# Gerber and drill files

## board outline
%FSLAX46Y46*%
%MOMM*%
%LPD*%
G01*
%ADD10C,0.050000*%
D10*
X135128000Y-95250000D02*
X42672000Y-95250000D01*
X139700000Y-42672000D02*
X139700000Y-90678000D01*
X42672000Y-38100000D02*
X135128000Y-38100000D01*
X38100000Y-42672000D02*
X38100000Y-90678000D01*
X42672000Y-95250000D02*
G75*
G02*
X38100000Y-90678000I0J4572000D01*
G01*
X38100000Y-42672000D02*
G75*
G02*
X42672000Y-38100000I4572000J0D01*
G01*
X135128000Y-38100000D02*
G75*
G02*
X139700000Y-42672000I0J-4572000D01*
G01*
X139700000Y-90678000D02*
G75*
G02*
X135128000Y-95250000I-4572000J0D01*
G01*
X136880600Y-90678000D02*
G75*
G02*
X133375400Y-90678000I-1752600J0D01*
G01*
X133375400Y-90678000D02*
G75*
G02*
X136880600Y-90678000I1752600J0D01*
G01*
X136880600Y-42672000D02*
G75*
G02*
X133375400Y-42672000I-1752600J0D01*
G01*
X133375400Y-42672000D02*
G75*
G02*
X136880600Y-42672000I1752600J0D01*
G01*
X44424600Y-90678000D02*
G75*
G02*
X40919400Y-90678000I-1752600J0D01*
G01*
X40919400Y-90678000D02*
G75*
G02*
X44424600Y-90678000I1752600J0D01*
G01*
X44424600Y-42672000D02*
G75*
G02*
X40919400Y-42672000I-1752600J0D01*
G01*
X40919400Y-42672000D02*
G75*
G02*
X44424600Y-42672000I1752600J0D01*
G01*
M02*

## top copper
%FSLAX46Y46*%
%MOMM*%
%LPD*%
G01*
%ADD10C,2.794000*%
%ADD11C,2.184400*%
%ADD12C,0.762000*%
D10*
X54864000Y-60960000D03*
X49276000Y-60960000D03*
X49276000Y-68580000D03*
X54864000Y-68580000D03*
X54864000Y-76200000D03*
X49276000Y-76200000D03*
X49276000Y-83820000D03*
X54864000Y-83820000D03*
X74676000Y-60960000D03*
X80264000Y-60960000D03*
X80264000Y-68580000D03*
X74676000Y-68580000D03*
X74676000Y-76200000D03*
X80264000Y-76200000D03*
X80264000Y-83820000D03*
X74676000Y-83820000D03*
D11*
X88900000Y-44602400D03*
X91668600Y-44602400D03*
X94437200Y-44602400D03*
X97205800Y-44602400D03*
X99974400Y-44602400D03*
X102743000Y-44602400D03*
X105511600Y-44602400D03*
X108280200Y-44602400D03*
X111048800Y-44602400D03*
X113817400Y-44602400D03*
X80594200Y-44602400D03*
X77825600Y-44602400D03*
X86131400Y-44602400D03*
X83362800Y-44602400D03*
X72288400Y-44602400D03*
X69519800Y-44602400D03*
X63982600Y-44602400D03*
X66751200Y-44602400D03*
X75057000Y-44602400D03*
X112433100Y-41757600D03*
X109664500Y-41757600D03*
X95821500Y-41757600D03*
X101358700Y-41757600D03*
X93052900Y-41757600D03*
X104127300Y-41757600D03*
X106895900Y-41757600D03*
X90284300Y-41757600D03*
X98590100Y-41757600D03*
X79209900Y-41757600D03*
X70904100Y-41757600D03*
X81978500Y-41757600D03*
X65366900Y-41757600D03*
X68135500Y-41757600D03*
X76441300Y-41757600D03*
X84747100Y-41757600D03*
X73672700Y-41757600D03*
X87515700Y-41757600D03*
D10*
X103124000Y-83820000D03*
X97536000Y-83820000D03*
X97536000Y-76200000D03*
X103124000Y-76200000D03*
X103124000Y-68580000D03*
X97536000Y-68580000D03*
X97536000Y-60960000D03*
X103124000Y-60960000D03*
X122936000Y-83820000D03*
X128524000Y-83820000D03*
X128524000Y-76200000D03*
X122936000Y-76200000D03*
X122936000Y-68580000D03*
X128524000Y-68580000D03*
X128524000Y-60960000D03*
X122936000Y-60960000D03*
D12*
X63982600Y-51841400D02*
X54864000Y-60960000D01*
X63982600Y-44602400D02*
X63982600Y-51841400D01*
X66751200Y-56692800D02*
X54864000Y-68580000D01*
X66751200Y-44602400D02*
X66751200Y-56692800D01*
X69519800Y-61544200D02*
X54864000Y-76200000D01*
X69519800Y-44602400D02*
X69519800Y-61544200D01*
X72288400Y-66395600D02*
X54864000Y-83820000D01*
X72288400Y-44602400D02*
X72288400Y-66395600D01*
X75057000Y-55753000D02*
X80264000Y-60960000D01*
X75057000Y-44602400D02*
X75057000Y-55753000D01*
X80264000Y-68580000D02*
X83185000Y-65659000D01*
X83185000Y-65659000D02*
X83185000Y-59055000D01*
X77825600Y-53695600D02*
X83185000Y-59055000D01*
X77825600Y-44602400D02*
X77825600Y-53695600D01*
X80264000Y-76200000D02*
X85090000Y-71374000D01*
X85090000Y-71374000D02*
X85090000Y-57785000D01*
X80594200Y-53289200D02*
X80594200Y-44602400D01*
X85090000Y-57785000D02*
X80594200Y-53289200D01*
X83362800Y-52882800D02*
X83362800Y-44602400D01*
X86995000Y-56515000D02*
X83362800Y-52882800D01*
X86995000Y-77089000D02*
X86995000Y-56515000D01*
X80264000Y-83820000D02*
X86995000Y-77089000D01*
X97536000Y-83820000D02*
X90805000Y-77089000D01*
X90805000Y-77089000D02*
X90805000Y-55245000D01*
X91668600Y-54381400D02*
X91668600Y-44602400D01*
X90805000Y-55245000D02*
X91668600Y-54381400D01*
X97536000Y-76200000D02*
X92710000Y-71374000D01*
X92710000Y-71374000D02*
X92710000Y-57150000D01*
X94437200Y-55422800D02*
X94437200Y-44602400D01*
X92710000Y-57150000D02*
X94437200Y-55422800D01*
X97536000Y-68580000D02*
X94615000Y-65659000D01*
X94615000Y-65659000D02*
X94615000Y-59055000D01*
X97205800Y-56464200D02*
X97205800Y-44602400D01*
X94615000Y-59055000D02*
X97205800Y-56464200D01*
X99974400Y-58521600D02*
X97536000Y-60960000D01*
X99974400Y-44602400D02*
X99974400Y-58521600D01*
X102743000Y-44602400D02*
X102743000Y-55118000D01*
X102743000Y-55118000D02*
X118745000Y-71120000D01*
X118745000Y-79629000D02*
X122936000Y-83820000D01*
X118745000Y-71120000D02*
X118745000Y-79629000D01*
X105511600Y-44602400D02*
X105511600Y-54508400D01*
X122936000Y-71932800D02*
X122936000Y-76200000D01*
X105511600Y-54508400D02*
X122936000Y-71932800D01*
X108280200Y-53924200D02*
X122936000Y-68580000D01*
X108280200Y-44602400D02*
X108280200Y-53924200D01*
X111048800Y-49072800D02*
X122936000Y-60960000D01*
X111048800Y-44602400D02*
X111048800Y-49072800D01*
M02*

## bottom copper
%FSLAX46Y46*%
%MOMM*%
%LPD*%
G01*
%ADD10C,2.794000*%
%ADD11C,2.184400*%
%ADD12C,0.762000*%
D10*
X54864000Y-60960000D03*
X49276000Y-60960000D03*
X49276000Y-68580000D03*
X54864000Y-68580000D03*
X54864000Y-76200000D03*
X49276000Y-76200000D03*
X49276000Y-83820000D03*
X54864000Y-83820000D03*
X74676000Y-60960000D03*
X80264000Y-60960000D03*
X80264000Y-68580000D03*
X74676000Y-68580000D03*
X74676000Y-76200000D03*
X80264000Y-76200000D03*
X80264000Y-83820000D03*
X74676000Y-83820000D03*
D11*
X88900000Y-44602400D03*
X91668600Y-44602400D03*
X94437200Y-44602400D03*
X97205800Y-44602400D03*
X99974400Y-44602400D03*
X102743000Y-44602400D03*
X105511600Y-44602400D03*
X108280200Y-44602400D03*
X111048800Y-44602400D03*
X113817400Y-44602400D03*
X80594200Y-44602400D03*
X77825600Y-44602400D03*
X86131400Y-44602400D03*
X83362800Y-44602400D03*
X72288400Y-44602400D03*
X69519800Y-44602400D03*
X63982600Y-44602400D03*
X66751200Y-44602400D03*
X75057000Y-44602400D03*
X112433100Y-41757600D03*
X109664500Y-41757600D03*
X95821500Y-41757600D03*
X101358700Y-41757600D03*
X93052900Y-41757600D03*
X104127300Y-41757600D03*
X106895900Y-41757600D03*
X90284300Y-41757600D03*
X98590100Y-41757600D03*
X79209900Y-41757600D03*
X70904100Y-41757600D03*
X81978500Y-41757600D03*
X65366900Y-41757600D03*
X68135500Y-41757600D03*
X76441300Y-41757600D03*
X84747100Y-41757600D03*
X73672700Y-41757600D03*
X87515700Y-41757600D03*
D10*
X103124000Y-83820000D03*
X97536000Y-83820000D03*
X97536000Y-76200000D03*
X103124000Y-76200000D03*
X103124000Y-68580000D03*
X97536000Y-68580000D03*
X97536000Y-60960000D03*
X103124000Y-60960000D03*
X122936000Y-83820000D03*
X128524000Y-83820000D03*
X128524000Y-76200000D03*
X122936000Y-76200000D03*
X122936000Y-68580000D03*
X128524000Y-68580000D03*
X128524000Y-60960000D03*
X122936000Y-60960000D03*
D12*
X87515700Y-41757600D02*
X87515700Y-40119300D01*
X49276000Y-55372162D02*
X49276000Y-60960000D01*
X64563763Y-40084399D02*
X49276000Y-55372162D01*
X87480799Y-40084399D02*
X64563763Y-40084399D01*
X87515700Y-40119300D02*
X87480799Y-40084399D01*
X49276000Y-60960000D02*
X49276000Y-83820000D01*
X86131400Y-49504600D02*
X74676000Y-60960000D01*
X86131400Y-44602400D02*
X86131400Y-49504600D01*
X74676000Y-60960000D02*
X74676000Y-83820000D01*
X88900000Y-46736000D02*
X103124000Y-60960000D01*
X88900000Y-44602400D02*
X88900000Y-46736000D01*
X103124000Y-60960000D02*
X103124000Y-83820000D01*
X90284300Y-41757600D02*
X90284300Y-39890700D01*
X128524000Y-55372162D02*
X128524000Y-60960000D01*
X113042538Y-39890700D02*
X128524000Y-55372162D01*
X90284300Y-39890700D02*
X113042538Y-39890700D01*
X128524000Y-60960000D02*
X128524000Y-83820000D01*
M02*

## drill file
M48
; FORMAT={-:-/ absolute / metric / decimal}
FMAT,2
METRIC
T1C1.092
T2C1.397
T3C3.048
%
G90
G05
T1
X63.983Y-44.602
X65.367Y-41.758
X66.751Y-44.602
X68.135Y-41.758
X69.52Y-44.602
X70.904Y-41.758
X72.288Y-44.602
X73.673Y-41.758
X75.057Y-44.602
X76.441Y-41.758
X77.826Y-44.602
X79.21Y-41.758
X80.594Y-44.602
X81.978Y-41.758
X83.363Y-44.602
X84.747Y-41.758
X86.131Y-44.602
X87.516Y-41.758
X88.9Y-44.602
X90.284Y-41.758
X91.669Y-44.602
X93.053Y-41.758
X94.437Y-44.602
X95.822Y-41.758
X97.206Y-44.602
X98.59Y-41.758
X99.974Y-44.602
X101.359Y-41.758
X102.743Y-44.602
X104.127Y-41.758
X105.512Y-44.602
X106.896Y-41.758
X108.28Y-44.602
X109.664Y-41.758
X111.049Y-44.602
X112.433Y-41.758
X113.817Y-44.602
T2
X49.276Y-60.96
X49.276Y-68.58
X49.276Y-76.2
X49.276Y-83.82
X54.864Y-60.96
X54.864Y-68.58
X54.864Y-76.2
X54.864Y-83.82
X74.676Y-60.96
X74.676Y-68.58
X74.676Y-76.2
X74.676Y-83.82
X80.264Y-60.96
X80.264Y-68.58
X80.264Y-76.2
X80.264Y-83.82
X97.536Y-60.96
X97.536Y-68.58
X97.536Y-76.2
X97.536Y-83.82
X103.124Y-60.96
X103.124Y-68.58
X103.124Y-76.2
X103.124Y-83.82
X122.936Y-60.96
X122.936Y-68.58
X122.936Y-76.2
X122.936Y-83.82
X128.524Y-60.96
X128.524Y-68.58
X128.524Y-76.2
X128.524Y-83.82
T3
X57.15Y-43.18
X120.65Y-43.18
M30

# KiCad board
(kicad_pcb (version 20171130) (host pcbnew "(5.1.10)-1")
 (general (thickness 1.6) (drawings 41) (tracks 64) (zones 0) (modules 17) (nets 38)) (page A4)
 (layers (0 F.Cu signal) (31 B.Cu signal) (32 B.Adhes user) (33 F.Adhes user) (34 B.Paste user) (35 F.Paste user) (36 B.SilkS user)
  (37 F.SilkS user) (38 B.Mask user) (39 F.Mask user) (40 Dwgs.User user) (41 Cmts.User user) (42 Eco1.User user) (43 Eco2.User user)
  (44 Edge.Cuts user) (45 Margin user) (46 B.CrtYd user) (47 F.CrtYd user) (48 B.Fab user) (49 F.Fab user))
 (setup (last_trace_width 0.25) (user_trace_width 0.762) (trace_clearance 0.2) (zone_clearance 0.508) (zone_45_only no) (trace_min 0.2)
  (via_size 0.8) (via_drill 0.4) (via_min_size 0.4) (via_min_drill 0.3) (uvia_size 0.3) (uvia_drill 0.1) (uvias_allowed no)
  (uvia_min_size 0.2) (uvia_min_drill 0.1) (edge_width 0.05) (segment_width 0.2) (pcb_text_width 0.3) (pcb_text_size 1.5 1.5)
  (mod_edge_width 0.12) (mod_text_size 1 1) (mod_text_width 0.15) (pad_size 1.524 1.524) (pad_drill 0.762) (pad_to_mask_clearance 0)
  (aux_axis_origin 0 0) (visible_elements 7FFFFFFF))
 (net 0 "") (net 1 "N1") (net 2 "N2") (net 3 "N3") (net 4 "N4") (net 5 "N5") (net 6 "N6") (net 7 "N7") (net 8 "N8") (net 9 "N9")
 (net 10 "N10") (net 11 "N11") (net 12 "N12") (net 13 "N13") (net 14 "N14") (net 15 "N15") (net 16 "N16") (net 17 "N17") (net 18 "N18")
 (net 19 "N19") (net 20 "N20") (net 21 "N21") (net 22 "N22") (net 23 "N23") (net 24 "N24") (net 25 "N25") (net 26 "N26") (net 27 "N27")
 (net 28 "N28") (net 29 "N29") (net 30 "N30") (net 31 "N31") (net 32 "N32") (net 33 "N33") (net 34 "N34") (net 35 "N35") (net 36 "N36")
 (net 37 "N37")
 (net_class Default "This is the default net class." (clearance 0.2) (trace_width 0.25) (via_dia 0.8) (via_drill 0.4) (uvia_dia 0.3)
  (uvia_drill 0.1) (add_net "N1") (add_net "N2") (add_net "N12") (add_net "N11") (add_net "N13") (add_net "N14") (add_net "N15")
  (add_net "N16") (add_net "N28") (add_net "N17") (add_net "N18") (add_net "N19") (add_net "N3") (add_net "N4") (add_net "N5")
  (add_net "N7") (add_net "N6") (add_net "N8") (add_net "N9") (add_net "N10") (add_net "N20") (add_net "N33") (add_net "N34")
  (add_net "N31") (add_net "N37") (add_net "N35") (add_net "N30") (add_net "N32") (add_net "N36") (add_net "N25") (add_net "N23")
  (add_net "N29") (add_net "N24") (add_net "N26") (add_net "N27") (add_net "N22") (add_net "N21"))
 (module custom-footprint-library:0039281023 (layer F.Cu) (at 52.07 60.96 180)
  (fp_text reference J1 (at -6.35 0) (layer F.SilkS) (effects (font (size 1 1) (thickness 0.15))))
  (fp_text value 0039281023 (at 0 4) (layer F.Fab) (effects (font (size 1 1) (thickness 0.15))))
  (pad 1 thru_hole circle (at -2.794 0 180) (size 2.794 2.794) (drill 1.397) (layers *.Cu *.Mask) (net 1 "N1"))
  (pad 2 thru_hole circle (at 2.794 0 180) (size 2.794 2.794) (drill 1.397) (layers *.Cu *.Mask) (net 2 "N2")))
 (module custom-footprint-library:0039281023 (layer F.Cu) (at 52.07 68.58 180)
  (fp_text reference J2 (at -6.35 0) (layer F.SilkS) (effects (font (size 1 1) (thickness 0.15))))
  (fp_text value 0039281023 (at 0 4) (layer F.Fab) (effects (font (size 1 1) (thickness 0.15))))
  (pad 2 thru_hole circle (at 2.794 0 180) (size 2.794 2.794) (drill 1.397) (layers *.Cu *.Mask) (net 2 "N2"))
  (pad 1 thru_hole circle (at -2.794 0 180) (size 2.794 2.794) (drill 1.397) (layers *.Cu *.Mask) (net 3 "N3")))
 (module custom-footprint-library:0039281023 (layer F.Cu) (at 52.07 76.2 180)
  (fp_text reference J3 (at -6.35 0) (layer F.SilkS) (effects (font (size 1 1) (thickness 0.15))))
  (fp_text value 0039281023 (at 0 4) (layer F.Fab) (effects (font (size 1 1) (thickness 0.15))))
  (pad 1 thru_hole circle (at -2.794 0 180) (size 2.794 2.794) (drill 1.397) (layers *.Cu *.Mask) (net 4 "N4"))
  (pad 2 thru_hole circle (at 2.794 0 180) (size 2.794 2.794) (drill 1.397) (layers *.Cu *.Mask) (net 2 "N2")))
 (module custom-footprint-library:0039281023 (layer F.Cu) (at 52.07 83.82 180)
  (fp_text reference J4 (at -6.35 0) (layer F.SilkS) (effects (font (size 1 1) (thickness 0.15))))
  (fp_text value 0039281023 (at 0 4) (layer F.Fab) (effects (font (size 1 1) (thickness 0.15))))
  (pad 2 thru_hole circle (at 2.794 0 180) (size 2.794 2.794) (drill 1.397) (layers *.Cu *.Mask) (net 2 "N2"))
  (pad 1 thru_hole circle (at -2.794 0 180) (size 2.794 2.794) (drill 1.397) (layers *.Cu *.Mask) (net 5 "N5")))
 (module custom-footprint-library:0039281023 (layer F.Cu) (at 77.47 60.96 180)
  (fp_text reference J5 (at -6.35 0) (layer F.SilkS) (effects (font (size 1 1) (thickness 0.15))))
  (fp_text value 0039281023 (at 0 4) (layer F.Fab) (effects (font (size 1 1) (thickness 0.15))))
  (pad 2 thru_hole circle (at 2.794 0 180) (size 2.794 2.794) (drill 1.397) (layers *.Cu *.Mask) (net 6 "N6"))
  (pad 1 thru_hole circle (at -2.794 0 180) (size 2.794 2.794) (drill 1.397) (layers *.Cu *.Mask) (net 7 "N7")))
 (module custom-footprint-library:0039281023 (layer F.Cu) (at 77.47 68.58 180)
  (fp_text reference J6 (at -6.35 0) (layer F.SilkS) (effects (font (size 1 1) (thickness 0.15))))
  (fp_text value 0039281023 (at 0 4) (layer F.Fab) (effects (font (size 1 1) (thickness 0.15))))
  (pad 1 thru_hole circle (at -2.794 0 180) (size 2.794 2.794) (drill 1.397) (layers *.Cu *.Mask) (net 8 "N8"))
  (pad 2 thru_hole circle (at 2.794 0 180) (size 2.794 2.794) (drill 1.397) (layers *.Cu *.Mask) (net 6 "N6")))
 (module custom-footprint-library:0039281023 (layer F.Cu) (at 77.47 76.2 180)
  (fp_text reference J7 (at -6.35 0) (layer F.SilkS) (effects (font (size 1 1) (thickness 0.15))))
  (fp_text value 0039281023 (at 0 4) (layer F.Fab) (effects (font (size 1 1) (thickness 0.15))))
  (pad 2 thru_hole circle (at 2.794 0 180) (size 2.794 2.794) (drill 1.397) (layers *.Cu *.Mask) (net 6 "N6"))
  (pad 1 thru_hole circle (at -2.794 0 180) (size 2.794 2.794) (drill 1.397) (layers *.Cu *.Mask) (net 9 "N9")))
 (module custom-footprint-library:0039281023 (layer F.Cu) (at 77.47 83.82 180)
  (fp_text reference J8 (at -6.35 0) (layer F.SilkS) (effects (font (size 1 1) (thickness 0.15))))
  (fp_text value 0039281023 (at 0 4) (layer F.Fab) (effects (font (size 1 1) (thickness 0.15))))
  (pad 1 thru_hole circle (at -2.794 0 180) (size 2.794 2.794) (drill 1.397) (layers *.Cu *.Mask) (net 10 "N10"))
  (pad 2 thru_hole circle (at 2.794 0 180) (size 2.794 2.794) (drill 1.397) (layers *.Cu *.Mask) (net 6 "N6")))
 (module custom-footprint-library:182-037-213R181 (layer F.Cu) (at 88.9 43.18)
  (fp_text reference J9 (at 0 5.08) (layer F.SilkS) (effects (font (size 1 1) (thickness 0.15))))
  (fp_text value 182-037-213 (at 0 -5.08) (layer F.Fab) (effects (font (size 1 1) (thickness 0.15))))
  (pad 10 thru_hole circle (at 0 1.4224) (size 2.1844 2.1844) (drill 1.0922) (layers *.Cu *.Mask) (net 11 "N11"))
  (pad 11 thru_hole circle (at 2.7686 1.4224) (size 2.1844 2.1844) (drill 1.0922) (layers *.Cu *.Mask) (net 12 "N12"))
  (pad 12 thru_hole circle (at 5.5372 1.4224) (size 2.1844 2.1844) (drill 1.0922) (layers *.Cu *.Mask) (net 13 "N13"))
  (pad 13 thru_hole circle (at 8.3058 1.4224) (size 2.1844 2.1844) (drill 1.0922) (layers *.Cu *.Mask) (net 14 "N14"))
  (pad 14 thru_hole circle (at 11.0744 1.4224) (size 2.1844 2.1844) (drill 1.0922) (layers *.Cu *.Mask) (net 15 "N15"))
  (pad 15 thru_hole circle (at 13.843 1.4224) (size 2.1844 2.1844) (drill 1.0922) (layers *.Cu *.Mask) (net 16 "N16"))
  (pad 16 thru_hole circle (at 16.6116 1.4224) (size 2.1844 2.1844) (drill 1.0922) (layers *.Cu *.Mask) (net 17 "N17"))
  (pad 17 thru_hole circle (at 19.3802 1.4224) (size 2.1844 2.1844) (drill 1.0922) (layers *.Cu *.Mask) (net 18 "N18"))
  (pad 18 thru_hole circle (at 22.1488 1.4224) (size 2.1844 2.1844) (drill 1.0922) (layers *.Cu *.Mask) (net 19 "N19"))
  (pad 19 thru_hole circle (at 24.9174 1.4224) (size 2.1844 2.1844) (drill 1.0922) (layers *.Cu *.Mask) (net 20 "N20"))
  (pad 7 thru_hole circle (at -8.3058 1.4224) (size 2.1844 2.1844) (drill 1.0922) (layers *.Cu *.Mask) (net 9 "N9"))
  (pad 6 thru_hole circle (at -11.0744 1.4224) (size 2.1844 2.1844) (drill 1.0922) (layers *.Cu *.Mask) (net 8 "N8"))
  (pad 9 thru_hole circle (at -2.7686 1.4224) (size 2.1844 2.1844) (drill 1.0922) (layers *.Cu *.Mask) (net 6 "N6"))
  (pad 8 thru_hole circle (at -5.5372 1.4224) (size 2.1844 2.1844) (drill 1.0922) (layers *.Cu *.Mask) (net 10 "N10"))
  (pad 4 thru_hole circle (at -16.6116 1.4224) (size 2.1844 2.1844) (drill 1.0922) (layers *.Cu *.Mask) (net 5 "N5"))
  (pad 3 thru_hole circle (at -19.3802 1.4224) (size 2.1844 2.1844) (drill 1.0922) (layers *.Cu *.Mask) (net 4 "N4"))
  (pad 1 thru_hole circle (at -24.9174 1.4224) (size 2.1844 2.1844) (drill 1.0922) (layers *.Cu *.Mask) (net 1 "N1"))
  (pad 2 thru_hole circle (at -22.1488 1.4224) (size 2.1844 2.1844) (drill 1.0922) (layers *.Cu *.Mask) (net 3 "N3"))
  (pad 5 thru_hole circle (at -13.843 1.4224) (size 2.1844 2.1844) (drill 1.0922) (layers *.Cu *.Mask) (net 7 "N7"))
  (pad 37 thru_hole circle (at 23.5331 -1.4224) (size 2.1844 2.1844) (drill 1.0922) (layers *.Cu *.Mask) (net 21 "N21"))
  (pad 36 thru_hole circle (at 20.7645 -1.4224) (size 2.1844 2.1844) (drill 1.0922) (layers *.Cu *.Mask) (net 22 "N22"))
  (pad 31 thru_hole circle (at 6.9215 -1.4224) (size 2.1844 2.1844) (drill 1.0922) (layers *.Cu *.Mask) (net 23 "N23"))
  (pad 33 thru_hole circle (at 12.4587 -1.4224) (size 2.1844 2.1844) (drill 1.0922) (layers *.Cu *.Mask) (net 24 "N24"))
  (pad 30 thru_hole circle (at 4.1529 -1.4224) (size 2.1844 2.1844) (drill 1.0922) (layers *.Cu *.Mask) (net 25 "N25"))
  (pad 34 thru_hole circle (at 15.2273 -1.4224) (size 2.1844 2.1844) (drill 1.0922) (layers *.Cu *.Mask) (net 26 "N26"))
  (pad 35 thru_hole circle (at 17.9959 -1.4224) (size 2.1844 2.1844) (drill 1.0922) (layers *.Cu *.Mask) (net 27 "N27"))
  (pad 29 thru_hole circle (at 1.3843 -1.4224) (size 2.1844 2.1844) (drill 1.0922) (layers *.Cu *.Mask) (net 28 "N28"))
  (pad 32 thru_hole circle (at 9.6901 -1.4224) (size 2.1844 2.1844) (drill 1.0922) (layers *.Cu *.Mask) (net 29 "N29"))
  (pad 25 thru_hole circle (at -9.6901 -1.4224) (size 2.1844 2.1844) (drill 1.0922) (layers *.Cu *.Mask) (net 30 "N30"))
  (pad 22 thru_hole circle (at -17.9959 -1.4224) (size 2.1844 2.1844) (drill 1.0922) (layers *.Cu *.Mask) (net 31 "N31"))
  (pad 26 thru_hole circle (at -6.9215 -1.4224) (size 2.1844 2.1844) (drill 1.0922) (layers *.Cu *.Mask) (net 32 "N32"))
  (pad 20 thru_hole circle (at -23.5331 -1.4224) (size 2.1844 2.1844) (drill 1.0922) (layers *.Cu *.Mask) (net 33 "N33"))
  (pad 21 thru_hole circle (at -20.7645 -1.4224) (size 2.1844 2.1844) (drill 1.0922) (layers *.Cu *.Mask) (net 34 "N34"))
  (pad 24 thru_hole circle (at -12.4587 -1.4224) (size 2.1844 2.1844) (drill 1.0922) (layers *.Cu *.Mask) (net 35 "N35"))
  (pad 27 thru_hole circle (at -4.1529 -1.4224) (size 2.1844 2.1844) (drill 1.0922) (layers *.Cu *.Mask) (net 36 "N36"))
  (pad 23 thru_hole circle (at -15.2273 -1.4224) (size 2.1844 2.1844) (drill 1.0922) (layers *.Cu *.Mask) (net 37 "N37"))
  (pad 28 thru_hole circle (at -1.3843 -1.4224) (size 2.1844 2.1844) (drill 1.0922) (layers *.Cu *.Mask) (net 2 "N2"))
  (pad "" np_thru_hole circle (at 31.75 0) (size 3.048 3.048) (drill 3.048) (layers *.Cu *.Mask))
  (pad "" np_thru_hole circle (at -31.75 0) (size 3.048 3.048) (drill 3.048) (layers *.Cu *.Mask)))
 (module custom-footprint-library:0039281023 (layer F.Cu) (at 100.33 83.82)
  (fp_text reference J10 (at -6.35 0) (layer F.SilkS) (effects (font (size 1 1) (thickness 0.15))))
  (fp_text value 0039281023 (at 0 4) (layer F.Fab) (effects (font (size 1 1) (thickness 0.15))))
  (pad 2 thru_hole circle (at 2.794 0) (size 2.794 2.794) (drill 1.397) (layers *.Cu *.Mask) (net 11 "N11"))
  (pad 1 thru_hole circle (at -2.794 0) (size 2.794 2.794) (drill 1.397) (layers *.Cu *.Mask) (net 12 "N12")))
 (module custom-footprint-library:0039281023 (layer F.Cu) (at 100.33 76.2)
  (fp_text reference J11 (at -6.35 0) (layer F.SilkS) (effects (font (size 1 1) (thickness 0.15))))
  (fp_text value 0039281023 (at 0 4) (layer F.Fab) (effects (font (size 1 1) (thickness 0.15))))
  (pad 1 thru_hole circle (at -2.794 0) (size 2.794 2.794) (drill 1.397) (layers *.Cu *.Mask) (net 13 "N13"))
  (pad 2 thru_hole circle (at 2.794 0) (size 2.794 2.794) (drill 1.397) (layers *.Cu *.Mask) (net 11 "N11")))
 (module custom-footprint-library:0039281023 (layer F.Cu) (at 100.33 68.58)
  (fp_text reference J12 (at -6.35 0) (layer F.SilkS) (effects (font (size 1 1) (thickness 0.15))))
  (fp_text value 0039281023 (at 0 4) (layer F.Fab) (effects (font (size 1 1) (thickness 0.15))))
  (pad 2 thru_hole circle (at 2.794 0) (size 2.794 2.794) (drill 1.397) (layers *.Cu *.Mask) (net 11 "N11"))
  (pad 1 thru_hole circle (at -2.794 0) (size 2.794 2.794) (drill 1.397) (layers *.Cu *.Mask) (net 14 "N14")))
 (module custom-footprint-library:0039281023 (layer F.Cu) (at 100.33 60.96)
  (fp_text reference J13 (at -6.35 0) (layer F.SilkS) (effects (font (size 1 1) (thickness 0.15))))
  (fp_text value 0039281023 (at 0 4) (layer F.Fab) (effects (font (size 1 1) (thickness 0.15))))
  (pad 1 thru_hole circle (at -2.794 0) (size 2.794 2.794) (drill 1.397) (layers *.Cu *.Mask) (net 15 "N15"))
  (pad 2 thru_hole circle (at 2.794 0) (size 2.794 2.794) (drill 1.397) (layers *.Cu *.Mask) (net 11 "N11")))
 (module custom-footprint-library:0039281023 (layer F.Cu) (at 125.73 83.82)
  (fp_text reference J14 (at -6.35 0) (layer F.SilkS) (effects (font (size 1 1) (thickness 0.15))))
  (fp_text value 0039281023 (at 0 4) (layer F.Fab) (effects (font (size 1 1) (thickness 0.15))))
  (pad 1 thru_hole circle (at -2.794 0) (size 2.794 2.794) (drill 1.397) (layers *.Cu *.Mask) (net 16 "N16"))
  (pad 2 thru_hole circle (at 2.794 0) (size 2.794 2.794) (drill 1.397) (layers *.Cu *.Mask) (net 28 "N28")))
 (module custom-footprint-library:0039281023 (layer F.Cu) (at 125.73 76.2)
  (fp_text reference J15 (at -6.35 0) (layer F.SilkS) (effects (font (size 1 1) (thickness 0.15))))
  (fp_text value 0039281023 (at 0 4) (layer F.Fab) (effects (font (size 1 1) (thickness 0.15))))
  (pad 2 thru_hole circle (at 2.794 0) (size 2.794 2.794) (drill 1.397) (layers *.Cu *.Mask) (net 28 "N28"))
  (pad 1 thru_hole circle (at -2.794 0) (size 2.794 2.794) (drill 1.397) (layers *.Cu *.Mask) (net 17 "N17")))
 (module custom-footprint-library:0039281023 (layer F.Cu) (at 125.73 68.58)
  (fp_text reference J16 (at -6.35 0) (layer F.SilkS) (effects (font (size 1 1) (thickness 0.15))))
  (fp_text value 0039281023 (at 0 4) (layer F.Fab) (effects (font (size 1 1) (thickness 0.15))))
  (pad 1 thru_hole circle (at -2.794 0) (size 2.794 2.794) (drill 1.397) (layers *.Cu *.Mask) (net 18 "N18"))
  (pad 2 thru_hole circle (at 2.794 0) (size 2.794 2.794) (drill 1.397) (layers *.Cu *.Mask) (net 28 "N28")))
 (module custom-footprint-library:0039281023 (layer F.Cu) (at 125.73 60.96)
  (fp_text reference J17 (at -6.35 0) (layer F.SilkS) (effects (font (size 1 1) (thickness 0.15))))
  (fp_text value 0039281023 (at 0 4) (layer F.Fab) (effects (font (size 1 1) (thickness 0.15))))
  (pad 2 thru_hole circle (at 2.794 0) (size 2.794 2.794) (drill 1.397) (layers *.Cu *.Mask) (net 28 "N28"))
  (pad 1 thru_hole circle (at -2.794 0) (size 2.794 2.794) (drill 1.397) (layers *.Cu *.Mask) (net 19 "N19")))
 (gr_line (start 135.128 95.25) (end 42.672 95.25) (layer Edge.Cuts) (width 0.05))
 (gr_line (start 139.7 42.672) (end 139.7 90.678) (layer Edge.Cuts) (width 0.05))
 (gr_line (start 42.672 38.1) (end 135.128 38.1) (layer Edge.Cuts) (width 0.05))
 (gr_line (start 38.1 42.672) (end 38.1 90.678) (layer Edge.Cuts) (width 0.05))
 (gr_arc (start 42.672 90.678) (end 38.1 90.678) (angle -90) (layer Edge.Cuts) (width 0.05))
 (gr_arc (start 42.672 42.672) (end 42.672 38.1) (angle -90) (layer Edge.Cuts) (width 0.05))
 (gr_arc (start 135.128 42.672) (end 139.7 42.672) (angle -90) (layer Edge.Cuts) (width 0.05))
 (gr_arc (start 135.128 90.678) (end 135.128 95.25) (angle -90) (layer Edge.Cuts) (width 0.05))
 (gr_circle (center 135.128 90.678) (end 136.8806 90.678) (layer Edge.Cuts) (width 0.05))
 (gr_circle (center 135.128 42.672) (end 136.8806 42.672) (layer Edge.Cuts) (width 0.05))
 (gr_circle (center 42.672 90.678) (end 44.4246 90.678) (layer Edge.Cuts) (width 0.05))
 (gr_circle (center 42.672 42.672) (end 44.4246 42.672) (layer Edge.Cuts) (width 0.05))
 (segment (start 63.9826 51.8414) (end 54.864 60.96) (width 0.762) (layer F.Cu) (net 1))
 (segment (start 63.9826 44.6024) (end 63.9826 51.8414) (width 0.762) (layer F.Cu) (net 1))
 (segment (start 87.5157 41.7576) (end 87.5157 40.1193) (width 0.762) (layer B.Cu) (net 2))
 (segment (start 49.276 55.372162) (end 49.276 60.96) (width 0.762) (layer B.Cu) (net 2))
 (segment (start 64.563763 40.084399) (end 49.276 55.372162) (width 0.762) (layer B.Cu) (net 2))
 (segment (start 87.480799 40.084399) (end 64.563763 40.084399) (width 0.762) (layer B.Cu) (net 2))
 (segment (start 87.5157 40.1193) (end 87.480799 40.084399) (width 0.762) (layer B.Cu) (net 2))
 (segment (start 49.276 60.96) (end 49.276 83.82) (width 0.762) (layer B.Cu) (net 2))
 (segment (start 66.7512 56.6928) (end 54.864 68.58) (width 0.762) (layer F.Cu) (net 3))
 (segment (start 66.7512 44.6024) (end 66.7512 56.6928) (width 0.762) (layer F.Cu) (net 3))
 (segment (start 69.5198 61.5442) (end 54.864 76.2) (width 0.762) (layer F.Cu) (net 4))
 (segment (start 69.5198 44.6024) (end 69.5198 61.5442) (width 0.762) (layer F.Cu) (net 4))
 (segment (start 72.2884 66.3956) (end 54.864 83.82) (width 0.762) (layer F.Cu) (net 5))
 (segment (start 72.2884 44.6024) (end 72.2884 66.3956) (width 0.762) (layer F.Cu) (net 5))
 (segment (start 86.1314 49.5046) (end 74.676 60.96) (width 0.762) (layer B.Cu) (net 6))
 (segment (start 86.1314 44.6024) (end 86.1314 49.5046) (width 0.762) (layer B.Cu) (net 6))
 (segment (start 74.676 60.96) (end 74.676 83.82) (width 0.762) (layer B.Cu) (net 6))
 (segment (start 75.057 55.753) (end 80.264 60.96) (width 0.762) (layer F.Cu) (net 7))
 (segment (start 75.057 44.6024) (end 75.057 55.753) (width 0.762) (layer F.Cu) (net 7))
 (segment (start 80.264 68.58) (end 83.185 65.659) (width 0.762) (layer F.Cu) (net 8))
 (segment (start 83.185 65.659) (end 83.185 59.055) (width 0.762) (layer F.Cu) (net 8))
 (segment (start 77.8256 53.6956) (end 83.185 59.055) (width 0.762) (layer F.Cu) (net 8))
 (segment (start 77.8256 44.6024) (end 77.8256 53.6956) (width 0.762) (layer F.Cu) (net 8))
 (segment (start 80.264 76.2) (end 85.09 71.374) (width 0.762) (layer F.Cu) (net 9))
 (segment (start 85.09 71.374) (end 85.09 57.785) (width 0.762) (layer F.Cu) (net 9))
 (segment (start 80.5942 53.2892) (end 80.5942 44.6024) (width 0.762) (layer F.Cu) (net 9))
 (segment (start 85.09 57.785) (end 80.5942 53.2892) (width 0.762) (layer F.Cu) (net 9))
 (segment (start 83.3628 52.8828) (end 83.3628 44.6024) (width 0.762) (layer F.Cu) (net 10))
 (segment (start 86.995 56.515) (end 83.3628 52.8828) (width 0.762) (layer F.Cu) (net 10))
 (segment (start 86.995 77.089) (end 86.995 56.515) (width 0.762) (layer F.Cu) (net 10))
 (segment (start 80.264 83.82) (end 86.995 77.089) (width 0.762) (layer F.Cu) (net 10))
 (segment (start 88.9 46.736) (end 103.124 60.96) (width 0.762) (layer B.Cu) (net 11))
 (segment (start 88.9 44.6024) (end 88.9 46.736) (width 0.762) (layer B.Cu) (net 11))
 (segment (start 103.124 60.96) (end 103.124 83.82) (width 0.762) (layer B.Cu) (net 11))
 (segment (start 97.536 83.82) (end 90.805 77.089) (width 0.762) (layer F.Cu) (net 12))
 (segment (start 90.805 77.089) (end 90.805 55.245) (width 0.762) (layer F.Cu) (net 12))
 (segment (start 91.6686 54.3814) (end 91.6686 44.6024) (width 0.762) (layer F.Cu) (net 12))
 (segment (start 90.805 55.245) (end 91.6686 54.3814) (width 0.762) (layer F.Cu) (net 12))
 (segment (start 97.536 76.2) (end 92.71 71.374) (width 0.762) (layer F.Cu) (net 13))
 (segment (start 92.71 71.374) (end 92.71 57.15) (width 0.762) (layer F.Cu) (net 13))
 (segment (start 94.4372 55.4228) (end 94.4372 44.6024) (width 0.762) (layer F.Cu) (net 13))
 (segment (start 92.71 57.15) (end 94.4372 55.4228) (width 0.762) (layer F.Cu) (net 13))
 (segment (start 97.536 68.58) (end 94.615 65.659) (width 0.762) (layer F.Cu) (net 14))
 (segment (start 94.615 65.659) (end 94.615 59.055) (width 0.762) (layer F.Cu) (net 14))
 (segment (start 97.2058 56.4642) (end 97.2058 44.6024) (width 0.762) (layer F.Cu) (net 14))
 (segment (start 94.615 59.055) (end 97.2058 56.4642) (width 0.762) (layer F.Cu) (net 14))
 (segment (start 99.9744 58.5216) (end 97.536 60.96) (width 0.762) (layer F.Cu) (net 15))
 (segment (start 99.9744 44.6024) (end 99.9744 58.5216) (width 0.762) (layer F.Cu) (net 15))
 (segment (start 102.743 44.6024) (end 102.743 55.118) (width 0.762) (layer F.Cu) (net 16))
 (segment (start 102.743 55.118) (end 118.745 71.12) (width 0.762) (layer F.Cu) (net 16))
 (segment (start 118.745 79.629) (end 122.936 83.82) (width 0.762) (layer F.Cu) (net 16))
 (segment (start 118.745 71.12) (end 118.745 79.629) (width 0.762) (layer F.Cu) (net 16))
 (segment (start 105.5116 44.6024) (end 105.5116 54.5084) (width 0.762) (layer F.Cu) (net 17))
 (segment (start 122.936 71.9328) (end 122.936 76.2) (width 0.762) (layer F.Cu) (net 17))
 (segment (start 105.5116 54.5084) (end 122.936 71.9328) (width 0.762) (layer F.Cu) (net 17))
 (segment (start 108.2802 53.9242) (end 122.936 68.58) (width 0.762) (layer F.Cu) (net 18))
 (segment (start 108.2802 44.6024) (end 108.2802 53.9242) (width 0.762) (layer F.Cu) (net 18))
 (segment (start 111.0488 49.0728) (end 122.936 60.96) (width 0.762) (layer F.Cu) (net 19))
 (segment (start 111.0488 44.6024) (end 111.0488 49.0728) (width 0.762) (layer F.Cu) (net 19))
 (segment (start 90.2843 41.7576) (end 90.2843 39.8907) (width 0.762) (layer B.Cu) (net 28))
 (segment (start 128.524 55.372162) (end 128.524 60.96) (width 0.762) (layer B.Cu) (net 28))
 (segment (start 113.042538 39.8907) (end 128.524 55.372162) (width 0.762) (layer B.Cu) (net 28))
 (segment (start 90.2843 39.8907) (end 113.042538 39.8907) (width 0.762) (layer B.Cu) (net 28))
 (segment (start 128.524 60.96) (end 128.524 83.82) (width 0.762) (layer B.Cu) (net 28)))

